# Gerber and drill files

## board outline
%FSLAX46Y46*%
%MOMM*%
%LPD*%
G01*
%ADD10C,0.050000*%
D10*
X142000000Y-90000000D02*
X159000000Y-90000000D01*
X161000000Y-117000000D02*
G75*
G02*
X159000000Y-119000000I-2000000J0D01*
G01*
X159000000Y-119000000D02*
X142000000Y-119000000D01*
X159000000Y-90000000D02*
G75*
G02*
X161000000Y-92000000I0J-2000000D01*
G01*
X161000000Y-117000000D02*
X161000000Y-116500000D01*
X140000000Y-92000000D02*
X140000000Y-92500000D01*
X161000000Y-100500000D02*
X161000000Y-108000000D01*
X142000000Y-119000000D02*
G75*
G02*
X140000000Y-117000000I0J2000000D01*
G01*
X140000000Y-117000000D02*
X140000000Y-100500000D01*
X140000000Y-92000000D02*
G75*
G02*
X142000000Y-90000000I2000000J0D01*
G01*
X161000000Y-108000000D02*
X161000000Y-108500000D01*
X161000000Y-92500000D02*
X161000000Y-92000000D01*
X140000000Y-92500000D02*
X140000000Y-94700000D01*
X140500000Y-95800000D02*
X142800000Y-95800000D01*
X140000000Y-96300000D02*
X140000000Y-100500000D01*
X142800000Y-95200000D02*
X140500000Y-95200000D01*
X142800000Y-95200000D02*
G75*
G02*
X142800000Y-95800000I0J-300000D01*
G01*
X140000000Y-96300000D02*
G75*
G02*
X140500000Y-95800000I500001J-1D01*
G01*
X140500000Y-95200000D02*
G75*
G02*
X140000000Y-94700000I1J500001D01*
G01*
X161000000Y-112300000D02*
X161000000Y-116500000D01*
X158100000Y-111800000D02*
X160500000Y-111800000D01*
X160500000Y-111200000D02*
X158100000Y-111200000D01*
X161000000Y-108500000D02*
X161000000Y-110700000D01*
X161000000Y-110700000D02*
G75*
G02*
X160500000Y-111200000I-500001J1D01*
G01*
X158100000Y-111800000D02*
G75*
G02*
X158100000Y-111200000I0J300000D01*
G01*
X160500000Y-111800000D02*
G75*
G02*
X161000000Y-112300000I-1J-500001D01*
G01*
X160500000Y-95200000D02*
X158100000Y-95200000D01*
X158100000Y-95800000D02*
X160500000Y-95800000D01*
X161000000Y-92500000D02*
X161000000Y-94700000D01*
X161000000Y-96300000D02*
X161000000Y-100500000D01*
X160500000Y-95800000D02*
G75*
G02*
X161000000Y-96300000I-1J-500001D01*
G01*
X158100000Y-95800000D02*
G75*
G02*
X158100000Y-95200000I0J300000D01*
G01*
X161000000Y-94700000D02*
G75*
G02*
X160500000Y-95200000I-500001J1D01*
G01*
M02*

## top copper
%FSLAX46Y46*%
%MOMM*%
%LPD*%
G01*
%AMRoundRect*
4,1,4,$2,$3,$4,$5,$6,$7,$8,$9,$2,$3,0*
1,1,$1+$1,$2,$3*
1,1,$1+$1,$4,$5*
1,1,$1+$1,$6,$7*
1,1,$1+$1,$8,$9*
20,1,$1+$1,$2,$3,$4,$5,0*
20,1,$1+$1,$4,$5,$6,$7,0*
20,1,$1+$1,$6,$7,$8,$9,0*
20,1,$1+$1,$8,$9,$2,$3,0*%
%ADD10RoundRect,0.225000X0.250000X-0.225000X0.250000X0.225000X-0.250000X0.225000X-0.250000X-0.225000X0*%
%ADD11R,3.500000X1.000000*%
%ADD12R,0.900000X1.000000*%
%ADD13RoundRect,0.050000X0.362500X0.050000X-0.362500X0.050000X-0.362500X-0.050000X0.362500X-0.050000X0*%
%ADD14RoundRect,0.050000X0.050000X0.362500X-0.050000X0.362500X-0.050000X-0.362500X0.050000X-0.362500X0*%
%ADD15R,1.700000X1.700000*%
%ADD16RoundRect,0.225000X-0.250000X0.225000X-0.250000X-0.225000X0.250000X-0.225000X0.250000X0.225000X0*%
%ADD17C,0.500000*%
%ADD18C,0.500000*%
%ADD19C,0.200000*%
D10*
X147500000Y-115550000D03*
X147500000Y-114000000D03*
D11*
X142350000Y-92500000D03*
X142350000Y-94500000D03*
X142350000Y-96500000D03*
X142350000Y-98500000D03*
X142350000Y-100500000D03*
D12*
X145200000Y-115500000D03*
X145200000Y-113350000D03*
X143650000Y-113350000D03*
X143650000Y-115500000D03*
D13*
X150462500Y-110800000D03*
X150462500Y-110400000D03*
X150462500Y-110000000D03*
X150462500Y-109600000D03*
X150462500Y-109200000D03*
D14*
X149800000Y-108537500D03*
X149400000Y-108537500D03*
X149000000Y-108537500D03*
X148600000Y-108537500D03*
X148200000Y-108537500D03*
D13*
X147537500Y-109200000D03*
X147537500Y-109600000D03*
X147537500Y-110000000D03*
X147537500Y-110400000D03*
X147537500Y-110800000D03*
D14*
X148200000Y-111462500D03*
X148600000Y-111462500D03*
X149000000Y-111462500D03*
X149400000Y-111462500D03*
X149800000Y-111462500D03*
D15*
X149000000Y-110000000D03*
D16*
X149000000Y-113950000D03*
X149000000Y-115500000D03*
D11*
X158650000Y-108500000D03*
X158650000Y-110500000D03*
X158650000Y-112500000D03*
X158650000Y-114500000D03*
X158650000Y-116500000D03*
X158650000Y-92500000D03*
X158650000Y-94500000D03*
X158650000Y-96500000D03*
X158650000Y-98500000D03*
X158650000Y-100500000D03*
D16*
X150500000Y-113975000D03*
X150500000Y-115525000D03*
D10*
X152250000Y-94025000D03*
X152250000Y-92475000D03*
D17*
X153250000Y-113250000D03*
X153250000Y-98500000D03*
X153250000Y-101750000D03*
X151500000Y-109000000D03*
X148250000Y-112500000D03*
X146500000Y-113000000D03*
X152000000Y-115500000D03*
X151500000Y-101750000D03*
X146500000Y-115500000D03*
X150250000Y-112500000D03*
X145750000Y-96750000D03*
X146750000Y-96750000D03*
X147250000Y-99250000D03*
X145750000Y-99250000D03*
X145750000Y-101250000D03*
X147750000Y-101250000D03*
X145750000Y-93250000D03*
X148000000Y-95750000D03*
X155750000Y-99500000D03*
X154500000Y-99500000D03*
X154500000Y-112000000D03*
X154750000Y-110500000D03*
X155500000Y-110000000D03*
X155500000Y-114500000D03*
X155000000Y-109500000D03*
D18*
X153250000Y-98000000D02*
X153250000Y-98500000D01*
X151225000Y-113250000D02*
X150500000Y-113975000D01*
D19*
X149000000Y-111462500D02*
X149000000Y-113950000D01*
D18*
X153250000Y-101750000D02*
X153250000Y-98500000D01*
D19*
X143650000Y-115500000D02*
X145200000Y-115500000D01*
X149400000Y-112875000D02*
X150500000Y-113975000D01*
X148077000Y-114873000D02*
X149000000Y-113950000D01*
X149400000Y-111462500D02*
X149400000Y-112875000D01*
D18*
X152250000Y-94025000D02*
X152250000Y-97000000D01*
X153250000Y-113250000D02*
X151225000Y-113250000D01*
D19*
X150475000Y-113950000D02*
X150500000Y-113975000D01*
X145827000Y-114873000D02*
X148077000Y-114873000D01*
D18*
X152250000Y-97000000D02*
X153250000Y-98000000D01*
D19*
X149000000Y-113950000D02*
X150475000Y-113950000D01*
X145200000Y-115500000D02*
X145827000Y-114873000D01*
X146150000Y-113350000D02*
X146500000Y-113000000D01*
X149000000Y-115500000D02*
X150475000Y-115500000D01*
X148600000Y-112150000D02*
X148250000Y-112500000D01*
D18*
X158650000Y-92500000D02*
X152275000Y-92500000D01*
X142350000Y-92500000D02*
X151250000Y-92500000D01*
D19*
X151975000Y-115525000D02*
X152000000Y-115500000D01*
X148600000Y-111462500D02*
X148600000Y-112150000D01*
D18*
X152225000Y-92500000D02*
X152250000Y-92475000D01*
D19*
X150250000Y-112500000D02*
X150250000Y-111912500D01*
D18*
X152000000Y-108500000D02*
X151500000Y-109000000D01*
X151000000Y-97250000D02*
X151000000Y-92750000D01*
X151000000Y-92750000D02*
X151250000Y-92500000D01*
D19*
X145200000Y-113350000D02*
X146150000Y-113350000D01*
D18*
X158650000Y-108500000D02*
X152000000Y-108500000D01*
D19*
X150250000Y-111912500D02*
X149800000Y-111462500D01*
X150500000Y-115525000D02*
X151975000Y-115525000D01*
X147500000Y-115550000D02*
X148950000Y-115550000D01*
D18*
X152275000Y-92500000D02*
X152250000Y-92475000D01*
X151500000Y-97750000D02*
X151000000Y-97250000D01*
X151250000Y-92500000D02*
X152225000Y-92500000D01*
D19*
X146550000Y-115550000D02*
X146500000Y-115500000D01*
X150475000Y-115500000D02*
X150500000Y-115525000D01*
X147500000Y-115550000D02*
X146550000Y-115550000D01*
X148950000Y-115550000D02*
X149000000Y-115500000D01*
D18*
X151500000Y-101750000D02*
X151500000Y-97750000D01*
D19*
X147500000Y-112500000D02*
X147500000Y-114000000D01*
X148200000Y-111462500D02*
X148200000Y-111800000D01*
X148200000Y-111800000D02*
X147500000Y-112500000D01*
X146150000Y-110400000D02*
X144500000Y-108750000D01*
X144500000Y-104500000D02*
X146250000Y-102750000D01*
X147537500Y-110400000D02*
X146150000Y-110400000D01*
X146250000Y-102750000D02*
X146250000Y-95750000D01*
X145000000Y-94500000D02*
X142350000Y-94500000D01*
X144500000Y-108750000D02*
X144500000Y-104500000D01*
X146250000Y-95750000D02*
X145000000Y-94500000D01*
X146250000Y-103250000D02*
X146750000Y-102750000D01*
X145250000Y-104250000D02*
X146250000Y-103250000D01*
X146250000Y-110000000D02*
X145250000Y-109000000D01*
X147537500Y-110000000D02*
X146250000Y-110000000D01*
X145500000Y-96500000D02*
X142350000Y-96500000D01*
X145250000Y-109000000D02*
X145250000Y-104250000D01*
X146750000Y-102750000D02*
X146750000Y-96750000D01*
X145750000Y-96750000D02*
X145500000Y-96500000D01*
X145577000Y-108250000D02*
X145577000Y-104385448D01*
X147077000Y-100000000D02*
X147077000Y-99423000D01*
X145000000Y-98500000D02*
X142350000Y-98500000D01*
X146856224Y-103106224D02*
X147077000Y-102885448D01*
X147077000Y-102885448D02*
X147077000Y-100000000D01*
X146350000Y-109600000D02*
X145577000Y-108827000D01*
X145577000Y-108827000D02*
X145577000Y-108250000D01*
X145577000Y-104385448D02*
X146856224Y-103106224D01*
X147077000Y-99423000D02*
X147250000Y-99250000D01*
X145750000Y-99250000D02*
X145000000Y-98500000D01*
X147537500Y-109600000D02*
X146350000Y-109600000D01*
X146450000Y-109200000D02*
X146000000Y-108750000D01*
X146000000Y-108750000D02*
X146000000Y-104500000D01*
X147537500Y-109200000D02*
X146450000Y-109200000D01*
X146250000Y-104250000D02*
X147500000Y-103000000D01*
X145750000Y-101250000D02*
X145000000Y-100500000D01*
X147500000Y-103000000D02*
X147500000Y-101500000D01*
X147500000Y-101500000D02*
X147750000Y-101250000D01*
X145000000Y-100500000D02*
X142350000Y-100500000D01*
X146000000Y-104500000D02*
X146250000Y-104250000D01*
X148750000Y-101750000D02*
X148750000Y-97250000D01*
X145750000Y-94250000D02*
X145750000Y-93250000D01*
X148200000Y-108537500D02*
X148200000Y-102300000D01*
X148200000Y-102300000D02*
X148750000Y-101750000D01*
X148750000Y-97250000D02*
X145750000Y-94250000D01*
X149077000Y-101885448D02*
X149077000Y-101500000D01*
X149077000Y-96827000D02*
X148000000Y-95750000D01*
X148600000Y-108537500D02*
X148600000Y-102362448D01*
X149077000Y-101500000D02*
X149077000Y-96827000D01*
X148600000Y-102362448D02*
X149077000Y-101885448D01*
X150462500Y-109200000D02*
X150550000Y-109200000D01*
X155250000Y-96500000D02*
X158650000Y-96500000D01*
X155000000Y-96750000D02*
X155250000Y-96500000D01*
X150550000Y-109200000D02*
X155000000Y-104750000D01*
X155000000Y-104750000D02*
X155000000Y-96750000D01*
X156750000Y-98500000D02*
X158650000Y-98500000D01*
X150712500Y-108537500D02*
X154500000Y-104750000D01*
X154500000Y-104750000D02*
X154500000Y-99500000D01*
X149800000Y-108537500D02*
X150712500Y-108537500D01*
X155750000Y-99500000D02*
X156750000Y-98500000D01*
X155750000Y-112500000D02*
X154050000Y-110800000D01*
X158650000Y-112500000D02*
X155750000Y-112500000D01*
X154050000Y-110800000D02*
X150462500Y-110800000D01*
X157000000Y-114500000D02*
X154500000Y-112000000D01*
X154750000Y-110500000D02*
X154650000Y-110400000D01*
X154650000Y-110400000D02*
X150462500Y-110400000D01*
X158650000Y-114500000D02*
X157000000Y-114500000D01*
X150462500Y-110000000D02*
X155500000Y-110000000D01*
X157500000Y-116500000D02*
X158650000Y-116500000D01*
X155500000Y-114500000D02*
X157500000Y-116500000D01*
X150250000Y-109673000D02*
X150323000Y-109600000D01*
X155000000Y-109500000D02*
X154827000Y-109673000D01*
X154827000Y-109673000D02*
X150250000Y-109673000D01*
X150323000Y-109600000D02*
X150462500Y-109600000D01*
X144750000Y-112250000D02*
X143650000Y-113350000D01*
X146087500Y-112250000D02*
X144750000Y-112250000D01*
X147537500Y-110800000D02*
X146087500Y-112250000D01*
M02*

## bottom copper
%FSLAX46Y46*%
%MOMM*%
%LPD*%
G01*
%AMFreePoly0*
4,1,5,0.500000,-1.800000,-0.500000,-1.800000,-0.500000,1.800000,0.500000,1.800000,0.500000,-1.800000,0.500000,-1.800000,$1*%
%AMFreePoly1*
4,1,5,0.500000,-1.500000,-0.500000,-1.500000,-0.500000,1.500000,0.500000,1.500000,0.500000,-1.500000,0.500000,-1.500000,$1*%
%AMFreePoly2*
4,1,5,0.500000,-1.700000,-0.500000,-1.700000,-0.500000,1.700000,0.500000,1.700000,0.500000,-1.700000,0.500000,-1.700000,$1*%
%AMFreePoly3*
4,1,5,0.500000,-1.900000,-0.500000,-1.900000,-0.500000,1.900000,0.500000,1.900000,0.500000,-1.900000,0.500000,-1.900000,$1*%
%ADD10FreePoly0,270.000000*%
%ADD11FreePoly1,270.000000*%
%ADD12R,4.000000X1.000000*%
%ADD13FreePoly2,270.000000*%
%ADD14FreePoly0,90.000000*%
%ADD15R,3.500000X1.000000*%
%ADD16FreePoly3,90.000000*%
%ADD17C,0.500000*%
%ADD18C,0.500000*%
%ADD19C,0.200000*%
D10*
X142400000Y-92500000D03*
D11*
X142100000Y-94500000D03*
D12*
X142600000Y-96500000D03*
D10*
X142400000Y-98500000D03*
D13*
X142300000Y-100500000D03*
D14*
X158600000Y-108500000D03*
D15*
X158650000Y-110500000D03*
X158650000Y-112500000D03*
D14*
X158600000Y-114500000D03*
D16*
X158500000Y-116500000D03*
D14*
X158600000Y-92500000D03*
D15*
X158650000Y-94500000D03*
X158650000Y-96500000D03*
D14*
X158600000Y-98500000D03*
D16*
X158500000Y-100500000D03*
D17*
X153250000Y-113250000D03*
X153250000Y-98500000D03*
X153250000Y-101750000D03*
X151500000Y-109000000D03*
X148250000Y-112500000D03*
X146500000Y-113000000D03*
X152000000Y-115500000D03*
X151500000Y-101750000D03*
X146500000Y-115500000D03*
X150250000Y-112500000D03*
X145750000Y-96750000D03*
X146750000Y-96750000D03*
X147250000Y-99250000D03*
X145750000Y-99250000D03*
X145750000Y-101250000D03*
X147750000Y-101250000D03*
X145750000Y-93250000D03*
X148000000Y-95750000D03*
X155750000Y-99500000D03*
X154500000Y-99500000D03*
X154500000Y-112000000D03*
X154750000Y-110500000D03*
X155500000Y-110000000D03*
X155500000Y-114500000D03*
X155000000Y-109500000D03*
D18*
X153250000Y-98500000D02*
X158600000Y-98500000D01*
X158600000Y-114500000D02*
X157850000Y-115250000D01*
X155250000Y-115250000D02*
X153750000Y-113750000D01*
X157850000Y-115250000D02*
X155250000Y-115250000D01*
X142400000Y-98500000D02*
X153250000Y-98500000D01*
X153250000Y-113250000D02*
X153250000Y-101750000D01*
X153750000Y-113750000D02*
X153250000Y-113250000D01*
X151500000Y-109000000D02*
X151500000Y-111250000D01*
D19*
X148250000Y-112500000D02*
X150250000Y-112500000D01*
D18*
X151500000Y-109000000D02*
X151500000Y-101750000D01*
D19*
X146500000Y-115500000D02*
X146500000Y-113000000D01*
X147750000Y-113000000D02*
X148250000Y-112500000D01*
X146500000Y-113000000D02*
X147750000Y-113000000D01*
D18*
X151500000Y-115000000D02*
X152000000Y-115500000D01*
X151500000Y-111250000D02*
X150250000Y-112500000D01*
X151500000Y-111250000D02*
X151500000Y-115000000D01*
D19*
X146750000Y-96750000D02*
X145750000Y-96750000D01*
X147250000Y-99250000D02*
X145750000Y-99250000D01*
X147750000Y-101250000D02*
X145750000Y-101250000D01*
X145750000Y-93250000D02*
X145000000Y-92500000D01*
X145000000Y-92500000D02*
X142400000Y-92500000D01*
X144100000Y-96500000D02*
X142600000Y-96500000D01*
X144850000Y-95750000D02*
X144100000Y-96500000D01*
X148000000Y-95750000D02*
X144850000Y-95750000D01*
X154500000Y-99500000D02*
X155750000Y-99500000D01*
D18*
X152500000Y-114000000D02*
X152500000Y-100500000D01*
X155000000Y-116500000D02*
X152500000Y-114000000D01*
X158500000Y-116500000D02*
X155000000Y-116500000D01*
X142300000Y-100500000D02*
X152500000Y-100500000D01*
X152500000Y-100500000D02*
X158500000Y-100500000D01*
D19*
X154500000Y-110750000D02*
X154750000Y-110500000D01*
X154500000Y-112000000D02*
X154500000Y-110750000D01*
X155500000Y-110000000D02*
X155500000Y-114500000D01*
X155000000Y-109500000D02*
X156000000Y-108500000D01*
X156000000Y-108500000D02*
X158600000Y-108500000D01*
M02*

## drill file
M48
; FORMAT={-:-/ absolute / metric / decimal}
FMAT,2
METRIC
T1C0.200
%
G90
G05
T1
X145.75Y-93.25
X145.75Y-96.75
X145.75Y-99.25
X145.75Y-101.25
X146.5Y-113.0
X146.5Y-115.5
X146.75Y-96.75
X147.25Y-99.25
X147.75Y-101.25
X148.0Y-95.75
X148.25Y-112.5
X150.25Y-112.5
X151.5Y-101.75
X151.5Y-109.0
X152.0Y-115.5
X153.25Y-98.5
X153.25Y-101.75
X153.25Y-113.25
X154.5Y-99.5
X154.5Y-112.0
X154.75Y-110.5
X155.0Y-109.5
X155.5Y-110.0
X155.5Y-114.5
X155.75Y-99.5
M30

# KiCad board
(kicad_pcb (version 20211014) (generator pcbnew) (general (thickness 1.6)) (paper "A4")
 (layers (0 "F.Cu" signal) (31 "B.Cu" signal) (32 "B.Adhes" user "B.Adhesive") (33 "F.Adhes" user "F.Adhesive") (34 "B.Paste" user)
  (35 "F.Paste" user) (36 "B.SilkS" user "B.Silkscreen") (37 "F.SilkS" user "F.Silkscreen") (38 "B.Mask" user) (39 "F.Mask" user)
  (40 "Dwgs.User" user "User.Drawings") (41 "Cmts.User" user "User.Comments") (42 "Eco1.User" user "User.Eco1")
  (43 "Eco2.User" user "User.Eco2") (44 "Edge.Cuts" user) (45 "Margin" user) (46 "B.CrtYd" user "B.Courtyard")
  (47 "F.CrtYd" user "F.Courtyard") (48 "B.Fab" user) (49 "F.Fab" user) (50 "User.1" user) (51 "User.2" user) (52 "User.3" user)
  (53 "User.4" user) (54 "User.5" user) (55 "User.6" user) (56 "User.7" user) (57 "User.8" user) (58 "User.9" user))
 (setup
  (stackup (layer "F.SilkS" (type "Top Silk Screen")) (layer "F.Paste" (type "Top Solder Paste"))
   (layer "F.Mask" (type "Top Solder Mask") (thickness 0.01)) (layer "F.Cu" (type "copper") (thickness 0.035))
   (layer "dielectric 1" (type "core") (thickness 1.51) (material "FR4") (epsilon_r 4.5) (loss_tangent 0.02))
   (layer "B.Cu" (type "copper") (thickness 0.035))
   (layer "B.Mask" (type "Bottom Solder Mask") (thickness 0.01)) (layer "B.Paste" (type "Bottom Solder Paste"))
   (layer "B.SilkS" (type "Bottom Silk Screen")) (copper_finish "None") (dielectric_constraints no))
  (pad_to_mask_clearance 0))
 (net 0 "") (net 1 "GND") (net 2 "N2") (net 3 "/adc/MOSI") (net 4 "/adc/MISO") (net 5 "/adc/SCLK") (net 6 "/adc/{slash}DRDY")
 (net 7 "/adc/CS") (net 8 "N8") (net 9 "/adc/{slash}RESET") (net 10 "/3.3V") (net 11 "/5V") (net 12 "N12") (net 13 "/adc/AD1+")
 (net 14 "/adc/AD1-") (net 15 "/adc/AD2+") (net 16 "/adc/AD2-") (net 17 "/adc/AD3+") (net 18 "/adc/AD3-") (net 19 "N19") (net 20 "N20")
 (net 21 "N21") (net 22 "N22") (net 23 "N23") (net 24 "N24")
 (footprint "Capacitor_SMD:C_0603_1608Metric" (layer "F.Cu") (at 147.5 114.775 90)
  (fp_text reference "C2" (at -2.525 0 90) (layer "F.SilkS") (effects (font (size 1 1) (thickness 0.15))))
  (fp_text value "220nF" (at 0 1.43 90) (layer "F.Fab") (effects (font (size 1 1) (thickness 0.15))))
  (pad "1" smd roundrect (at -0.775 0 90) (size 0.9 0.95) (layers "F.Cu" "F.Paste" "F.Mask") (roundrect_rratio 0.25) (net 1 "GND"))
  (pad "2" smd roundrect (at 0.775 0 90) (size 0.9 0.95) (layers "F.Cu" "F.Paste" "F.Mask") (roundrect_rratio 0.25) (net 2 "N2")))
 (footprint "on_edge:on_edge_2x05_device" (layer "F.Cu") (at 140 96.5 -90)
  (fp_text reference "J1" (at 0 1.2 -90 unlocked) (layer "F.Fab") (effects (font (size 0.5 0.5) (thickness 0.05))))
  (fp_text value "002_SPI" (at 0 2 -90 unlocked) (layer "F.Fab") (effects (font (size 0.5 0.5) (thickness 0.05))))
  (fp_line (start -4 0) (end -1.8 0) (layer "Edge.Cuts") (width 0.05))
  (fp_line (start -0.7 -0.5) (end -0.7 -2.8) (layer "Edge.Cuts") (width 0.05))
  (fp_line (start -0.2 0) (end 4 0) (layer "Edge.Cuts") (width 0.05))
  (fp_line (start -1.3 -2.8) (end -1.3 -0.5) (layer "Edge.Cuts") (width 0.05))
  (fp_arc (start -1.3 -2.8) (mid -1 -3.1) (end -0.7 -2.8) (layer "Edge.Cuts") (width 0.05))
  (fp_arc (start -0.2 0) (mid -0.553553 -0.146447) (end -0.7 -0.5) (layer "Edge.Cuts") (width 0.05))
  (fp_arc (start -1.3 -0.5) (mid -1.446447 -0.146447) (end -1.8 0) (layer "Edge.Cuts") (width 0.05))
  (pad "1" smd rect (at -4 -2.35 90) (size 1 3.5) (layers "F.Cu" "F.Mask") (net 1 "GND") (zone_connect 0))
  (pad "2" smd rect (at -2 -2.35 270) (size 1 3.5) (layers "F.Cu" "F.Mask") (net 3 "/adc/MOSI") (zone_connect 0))
  (pad "3" smd rect (at 0 -2.35 270) (size 1 3.5) (layers "F.Cu" "F.Mask") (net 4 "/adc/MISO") (zone_connect 0))
  (pad "4" smd rect (at 2 -2.35 90) (size 1 3.5) (layers "F.Cu" "F.Mask") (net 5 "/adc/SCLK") (zone_connect 0))
  (pad "5" smd rect (at 4 -2.35 90) (size 1 3.5) (layers "F.Cu" "F.Mask") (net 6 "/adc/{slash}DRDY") (zone_connect 0))
  (pad "6" smd custom (at -4 -2.4 270) (size 1 3.6) (layers "B.Cu" "B.Mask") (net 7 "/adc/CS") (zone_connect 0)
   (options (clearance outline) (anchor rect)) (primitives))
  (pad "7" smd custom (at -2 -2.1 270) (size 1 3) (layers "B.Cu" "B.Mask") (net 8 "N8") (zone_connect 0)
   (options (clearance outline) (anchor rect)) (primitives))
  (pad "8" smd rect (at 0 -2.6 270) (size 1 4) (layers "B.Cu" "B.Mask") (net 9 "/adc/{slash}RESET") (zone_connect 0))
  (pad "9" smd custom (at 2 -2.4 270) (size 1 3.6) (layers "B.Cu" "B.Mask") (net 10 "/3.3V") (zone_connect 0)
   (options (clearance outline) (anchor rect)) (primitives))
  (pad "10" smd custom (at 4 -2.3 270) (size 1 3.4) (layers "B.Cu" "B.Mask") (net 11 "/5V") (zone_connect 0)
   (options (clearance outline) (anchor rect)) (primitives)))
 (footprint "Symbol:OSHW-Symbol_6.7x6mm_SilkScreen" (layer "F.Cu") (at 143.4 108.6)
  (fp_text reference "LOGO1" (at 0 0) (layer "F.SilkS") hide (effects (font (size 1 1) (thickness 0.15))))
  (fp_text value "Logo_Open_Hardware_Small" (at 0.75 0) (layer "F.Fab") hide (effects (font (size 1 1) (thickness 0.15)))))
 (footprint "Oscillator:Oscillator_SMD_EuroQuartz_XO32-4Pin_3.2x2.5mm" (layer "F.Cu") (at 144.425 114.425 180)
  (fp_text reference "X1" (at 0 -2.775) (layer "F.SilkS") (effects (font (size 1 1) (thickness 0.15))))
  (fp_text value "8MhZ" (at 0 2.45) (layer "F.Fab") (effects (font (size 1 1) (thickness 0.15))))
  (pad "1" smd rect (at -0.775 -1.075 90) (size 1 0.9) (layers "F.Cu" "F.Paste" "F.Mask") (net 10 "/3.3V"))
  (pad "2" smd rect (at -0.775 1.075 90) (size 1 0.9) (layers "F.Cu" "F.Paste" "F.Mask") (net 1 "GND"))
  (pad "3" smd rect (at 0.775 1.075 90) (size 1 0.9) (layers "F.Cu" "F.Paste" "F.Mask") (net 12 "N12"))
  (pad "4" smd rect (at 0.775 -1.075 90) (size 1 0.9) (layers "F.Cu" "F.Paste" "F.Mask") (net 10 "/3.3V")))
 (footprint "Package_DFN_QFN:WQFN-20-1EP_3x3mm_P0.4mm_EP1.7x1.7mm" (layer "F.Cu") (at 149 110 180)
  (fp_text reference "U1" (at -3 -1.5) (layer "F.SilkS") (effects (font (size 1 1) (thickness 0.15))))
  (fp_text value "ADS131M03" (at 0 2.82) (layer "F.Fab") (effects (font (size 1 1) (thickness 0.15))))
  (pad "" smd roundrect (at -0.425 0.425 180) (size 0.69 0.69) (layers "F.Paste") (roundrect_rratio 0.25))
  (pad "" smd roundrect (at 0.425 0.425 180) (size 0.69 0.69) (layers "F.Paste") (roundrect_rratio 0.25))
  (pad "" smd roundrect (at -0.425 -0.425 180) (size 0.69 0.69) (layers "F.Paste") (roundrect_rratio 0.25))
  (pad "" smd roundrect (at 0.425 -0.425 180) (size 0.69 0.69) (layers "F.Paste") (roundrect_rratio 0.25))
  (pad "1" smd roundrect (at -1.4625 -0.8 180) (size 0.825 0.2) (layers "F.Cu" "F.Paste" "F.Mask") (roundrect_rratio 0.25)
   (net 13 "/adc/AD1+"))
  (pad "2" smd roundrect (at -1.4625 -0.4 180) (size 0.825 0.2) (layers "F.Cu" "F.Paste" "F.Mask") (roundrect_rratio 0.25)
   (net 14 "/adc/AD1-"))
  (pad "3" smd roundrect (at -1.4625 0 180) (size 0.825 0.2) (layers "F.Cu" "F.Paste" "F.Mask") (roundrect_rratio 0.25) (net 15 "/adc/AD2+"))
  (pad "4" smd roundrect (at -1.4625 0.4 180) (size 0.825 0.2) (layers "F.Cu" "F.Paste" "F.Mask") (roundrect_rratio 0.25)
   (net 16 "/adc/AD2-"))
  (pad "5" smd roundrect (at -1.4625 0.8 180) (size 0.825 0.2) (layers "F.Cu" "F.Paste" "F.Mask") (roundrect_rratio 0.25)
   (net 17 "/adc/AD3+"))
  (pad "6" smd roundrect (at -0.8 1.4625 180) (size 0.2 0.825) (layers "F.Cu" "F.Paste" "F.Mask") (roundrect_rratio 0.25)
   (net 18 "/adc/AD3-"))
  (pad "7" smd roundrect (at -0.4 1.4625 180) (size 0.2 0.825) (layers "F.Cu" "F.Paste" "F.Mask") (roundrect_rratio 0.25) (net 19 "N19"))
  (pad "8" smd roundrect (at 0 1.4625 180) (size 0.2 0.825) (layers "F.Cu" "F.Paste" "F.Mask") (roundrect_rratio 0.25) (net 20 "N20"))
  (pad "9" smd roundrect (at 0.4 1.4625 180) (size 0.2 0.825) (layers "F.Cu" "F.Paste" "F.Mask") (roundrect_rratio 0.25)
   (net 9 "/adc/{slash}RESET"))
  (pad "10" smd roundrect (at 0.8 1.4625 180) (size 0.2 0.825) (layers "F.Cu" "F.Paste" "F.Mask") (roundrect_rratio 0.25) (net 7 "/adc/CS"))
  (pad "11" smd roundrect (at 1.4625 0.8 180) (size 0.825 0.2) (layers "F.Cu" "F.Paste" "F.Mask") (roundrect_rratio 0.25)
   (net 6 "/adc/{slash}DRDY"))
  (pad "12" smd roundrect (at 1.4625 0.4 180) (size 0.825 0.2) (layers "F.Cu" "F.Paste" "F.Mask") (roundrect_rratio 0.25)
   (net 5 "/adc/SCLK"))
  (pad "13" smd roundrect (at 1.4625 0 180) (size 0.825 0.2) (layers "F.Cu" "F.Paste" "F.Mask") (roundrect_rratio 0.25) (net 4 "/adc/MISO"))
  (pad "14" smd roundrect (at 1.4625 -0.4 180) (size 0.825 0.2) (layers "F.Cu" "F.Paste" "F.Mask") (roundrect_rratio 0.25)
   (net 3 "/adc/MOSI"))
  (pad "15" smd roundrect (at 1.4625 -0.8 180) (size 0.825 0.2) (layers "F.Cu" "F.Paste" "F.Mask") (roundrect_rratio 0.25) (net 12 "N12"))
  (pad "16" smd roundrect (at 0.8 -1.4625 180) (size 0.2 0.825) (layers "F.Cu" "F.Paste" "F.Mask") (roundrect_rratio 0.25) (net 2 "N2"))
  (pad "17" smd roundrect (at 0.4 -1.4625 180) (size 0.2 0.825) (layers "F.Cu" "F.Paste" "F.Mask") (roundrect_rratio 0.25) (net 1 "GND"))
  (pad "18" smd roundrect (at 0 -1.4625 180) (size 0.2 0.825) (layers "F.Cu" "F.Paste" "F.Mask") (roundrect_rratio 0.25) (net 10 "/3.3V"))
  (pad "19" smd roundrect (at -0.4 -1.4625 180) (size 0.2 0.825) (layers "F.Cu" "F.Paste" "F.Mask") (roundrect_rratio 0.25) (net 10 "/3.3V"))
  (pad "20" smd roundrect (at -0.8 -1.4625 180) (size 0.2 0.825) (layers "F.Cu" "F.Paste" "F.Mask") (roundrect_rratio 0.25) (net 1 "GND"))
  (pad "21" smd rect (at 0 0 180) (size 1.7 1.7) (layers "F.Cu" "F.Mask")))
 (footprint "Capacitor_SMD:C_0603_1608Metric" (layer "F.Cu") (at 149 114.725 -90)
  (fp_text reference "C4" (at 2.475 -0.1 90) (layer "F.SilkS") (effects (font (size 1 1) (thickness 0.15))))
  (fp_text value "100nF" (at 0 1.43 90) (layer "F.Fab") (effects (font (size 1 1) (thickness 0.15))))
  (pad "1" smd roundrect (at -0.775 0 270) (size 0.9 0.95) (layers "F.Cu" "F.Paste" "F.Mask") (roundrect_rratio 0.25) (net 10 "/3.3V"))
  (pad "2" smd roundrect (at 0.775 0 270) (size 0.9 0.95) (layers "F.Cu" "F.Paste" "F.Mask") (roundrect_rratio 0.25) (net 1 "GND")))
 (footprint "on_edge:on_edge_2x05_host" (layer "F.Cu") (at 161 112.5 -90)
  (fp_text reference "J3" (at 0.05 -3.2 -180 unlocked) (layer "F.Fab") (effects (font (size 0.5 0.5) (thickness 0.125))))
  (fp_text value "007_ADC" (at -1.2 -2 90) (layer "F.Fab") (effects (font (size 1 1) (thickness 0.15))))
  (fp_line (start -0.2 0) (end 4 0) (layer "Edge.Cuts") (width 0.05))
  (fp_line (start -0.7 2.9) (end -0.7 0.5) (layer "Edge.Cuts") (width 0.05))
  (fp_line (start -1.3 0.5) (end -1.3 2.9) (layer "Edge.Cuts") (width 0.05))
  (fp_line (start -4 0) (end -1.8 0) (layer "Edge.Cuts") (width 0.05))
  (fp_arc (start -1.8 0) (mid -1.446447 0.146447) (end -1.3 0.5) (layer "Edge.Cuts") (width 0.05))
  (fp_arc (start -0.7 2.9) (mid -1 3.2) (end -1.3 2.9) (layer "Edge.Cuts") (width 0.05))
  (fp_arc (start -0.7 0.5) (mid -0.553553 0.146447) (end -0.2 0) (layer "Edge.Cuts") (width 0.05))
  (pad "1" smd rect (at -4 2.35 270) (size 1 3.5) (layers "F.Cu" "F.Mask") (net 1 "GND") (zone_connect 0))
  (pad "2" smd rect (at -2 2.35 270) (size 1 3.5) (layers "F.Cu" "F.Mask") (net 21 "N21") (zone_connect 0))
  (pad "3" smd rect (at 0 2.35 270) (size 1 3.5) (layers "F.Cu" "F.Mask") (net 13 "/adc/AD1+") (zone_connect 0))
  (pad "4" smd rect (at 2 2.35 270) (size 1 3.5) (layers "F.Cu" "F.Mask") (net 14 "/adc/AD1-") (zone_connect 0))
  (pad "5" smd rect (at 4 2.35 270) (size 1 3.5) (layers "F.Cu" "F.Mask") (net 15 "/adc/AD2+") (zone_connect 0))
  (pad "6" smd custom (at -4 2.4 90) (size 1 3.6) (layers "B.Cu" "B.Mask") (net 16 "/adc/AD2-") (zone_connect 0)
   (options (clearance outline) (anchor rect)) (primitives))
  (pad "7" smd rect (at -2 2.35 90) (size 1 3.5) (layers "B.Cu" "B.Mask") (zone_connect 0))
  (pad "8" smd rect (at 0 2.35 90) (size 1 3.5) (layers "B.Cu" "B.Mask") (zone_connect 0))
  (pad "9" smd custom (at 2 2.4 90) (size 1 3.6) (layers "B.Cu" "B.Mask") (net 10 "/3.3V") (zone_connect 0)
   (options (clearance outline) (anchor rect)) (primitives))
  (pad "10" smd custom (at 4 2.5 90) (size 1 3.8) (layers "B.Cu" "B.Mask") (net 11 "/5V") (zone_connect 0)
   (options (clearance outline) (anchor rect)) (primitives)))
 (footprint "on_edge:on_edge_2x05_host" (layer "F.Cu") (at 161 96.5 -90)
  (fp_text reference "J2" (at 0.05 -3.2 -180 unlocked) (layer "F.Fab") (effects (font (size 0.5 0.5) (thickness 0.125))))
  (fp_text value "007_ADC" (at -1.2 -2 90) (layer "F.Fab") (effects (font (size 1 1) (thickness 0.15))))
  (fp_line (start -1.3 0.5) (end -1.3 2.9) (layer "Edge.Cuts") (width 0.05))
  (fp_line (start -0.7 2.9) (end -0.7 0.5) (layer "Edge.Cuts") (width 0.05))
  (fp_line (start -4 0) (end -1.8 0) (layer "Edge.Cuts") (width 0.05))
  (fp_line (start -0.2 0) (end 4 0) (layer "Edge.Cuts") (width 0.05))
  (fp_arc (start -0.7 0.5) (mid -0.553553 0.146447) (end -0.2 0) (layer "Edge.Cuts") (width 0.05))
  (fp_arc (start -0.7 2.9) (mid -1 3.2) (end -1.3 2.9) (layer "Edge.Cuts") (width 0.05))
  (fp_arc (start -1.8 0) (mid -1.446447 0.146447) (end -1.3 0.5) (layer "Edge.Cuts") (width 0.05))
  (pad "1" smd rect (at -4 2.35 270) (size 1 3.5) (layers "F.Cu" "F.Mask") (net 1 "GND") (zone_connect 0))
  (pad "2" smd rect (at -2 2.35 270) (size 1 3.5) (layers "F.Cu" "F.Mask") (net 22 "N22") (zone_connect 0))
  (pad "3" smd rect (at 0 2.35 270) (size 1 3.5) (layers "F.Cu" "F.Mask") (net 17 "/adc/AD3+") (zone_connect 0))
  (pad "4" smd rect (at 2 2.35 270) (size 1 3.5) (layers "F.Cu" "F.Mask") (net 18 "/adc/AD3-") (zone_connect 0))
  (pad "5" smd rect (at 4 2.35 270) (size 1 3.5) (layers "F.Cu" "F.Mask") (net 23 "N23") (zone_connect 0))
  (pad "6" smd custom (at -4 2.4 90) (size 1 3.6) (layers "B.Cu" "B.Mask") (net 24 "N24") (zone_connect 0)
   (options (clearance outline) (anchor rect)) (primitives))
  (pad "7" smd rect (at -2 2.35 90) (size 1 3.5) (layers "B.Cu" "B.Mask") (zone_connect 0))
  (pad "8" smd rect (at 0 2.35 90) (size 1 3.5) (layers "B.Cu" "B.Mask") (zone_connect 0))
  (pad "9" smd custom (at 2 2.4 90) (size 1 3.6) (layers "B.Cu" "B.Mask") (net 10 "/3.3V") (zone_connect 0)
   (options (clearance outline) (anchor rect)) (primitives))
  (pad "10" smd custom (at 4 2.5 90) (size 1 3.8) (layers "B.Cu" "B.Mask") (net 11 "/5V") (zone_connect 0)
   (options (clearance outline) (anchor rect)) (primitives)))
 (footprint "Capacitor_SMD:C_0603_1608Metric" (layer "F.Cu") (at 150.5 114.75 -90)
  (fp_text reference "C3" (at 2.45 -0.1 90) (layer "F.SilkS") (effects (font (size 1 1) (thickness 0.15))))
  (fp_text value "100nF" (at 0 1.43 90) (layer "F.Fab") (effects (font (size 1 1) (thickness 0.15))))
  (pad "1" smd roundrect (at -0.775 0 270) (size 0.9 0.95) (layers "F.Cu" "F.Paste" "F.Mask") (roundrect_rratio 0.25) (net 10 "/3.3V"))
  (pad "2" smd roundrect (at 0.775 0 270) (size 0.9 0.95) (layers "F.Cu" "F.Paste" "F.Mask") (roundrect_rratio 0.25) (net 1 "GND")))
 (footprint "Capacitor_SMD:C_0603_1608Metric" (layer "F.Cu") (at 152.25 93.25 90)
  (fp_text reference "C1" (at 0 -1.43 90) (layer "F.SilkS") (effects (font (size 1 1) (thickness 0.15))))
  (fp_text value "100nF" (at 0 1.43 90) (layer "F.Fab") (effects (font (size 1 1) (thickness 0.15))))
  (pad "1" smd roundrect (at -0.775 0 90) (size 0.9 0.95) (layers "F.Cu" "F.Paste" "F.Mask") (roundrect_rratio 0.25) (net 10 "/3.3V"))
  (pad "2" smd roundrect (at 0.775 0 90) (size 0.9 0.95) (layers "F.Cu" "F.Paste" "F.Mask") (roundrect_rratio 0.25) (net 1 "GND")))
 (gr_line (start 142 90) (end 159 90) (layer "Edge.Cuts") (width 0.05))
 (gr_arc (start 161 117) (mid 160.414214 118.414214) (end 159 119) (layer "Edge.Cuts") (width 0.05))
 (gr_line (start 159 119) (end 142 119) (layer "Edge.Cuts") (width 0.05))
 (gr_arc (start 159 90) (mid 160.414214 90.585786) (end 161 92) (layer "Edge.Cuts") (width 0.05))
 (gr_line (start 161 117) (end 161 116.5) (layer "Edge.Cuts") (width 0.05))
 (gr_line (start 140 92) (end 140 92.5) (layer "Edge.Cuts") (width 0.05))
 (gr_line (start 161 100.5) (end 161 108) (layer "Edge.Cuts") (width 0.05))
 (gr_arc (start 142 119) (mid 140.585786 118.414214) (end 140 117) (layer "Edge.Cuts") (width 0.05))
 (gr_line (start 140 117) (end 140 100.5) (layer "Edge.Cuts") (width 0.05))
 (gr_arc (start 140 92) (mid 140.585786 90.585786) (end 142 90) (layer "Edge.Cuts") (width 0.05))
 (gr_line (start 161 108) (end 161 108.5) (layer "Edge.Cuts") (width 0.05))
 (gr_line (start 161 92.5) (end 161 92) (layer "Edge.Cuts") (width 0.05))
 (segment (start 153.25 98) (end 153.25 98.5) (width 0.5) (layer "F.Cu") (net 10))
 (segment (start 151.225 113.25) (end 150.5 113.975) (width 0.5) (layer "F.Cu") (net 10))
 (segment (start 149 111.4625) (end 149 113.95) (width 0.2) (layer "F.Cu") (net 10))
 (segment (start 153.25 101.75) (end 153.25 98.5) (width 0.5) (layer "F.Cu") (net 10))
 (segment (start 143.65 115.5) (end 145.2 115.5) (width 0.2) (layer "F.Cu") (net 10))
 (segment (start 149.4 112.875) (end 150.5 113.975) (width 0.2) (layer "F.Cu") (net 10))
 (segment (start 148.077 114.873) (end 149 113.95) (width 0.2) (layer "F.Cu") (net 10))
 (segment (start 149.4 111.4625) (end 149.4 112.875) (width 0.2) (layer "F.Cu") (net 10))
 (segment (start 152.25 94.025) (end 152.25 97) (width 0.5) (layer "F.Cu") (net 10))
 (segment (start 153.25 113.25) (end 151.225 113.25) (width 0.5) (layer "F.Cu") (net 10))
 (segment (start 150.475 113.95) (end 150.5 113.975) (width 0.2) (layer "F.Cu") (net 10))
 (segment (start 145.827 114.873) (end 148.077 114.873) (width 0.2) (layer "F.Cu") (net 10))
 (segment (start 152.25 97) (end 153.25 98) (width 0.5) (layer "F.Cu") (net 10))
 (segment (start 149 113.95) (end 150.475 113.95) (width 0.2) (layer "F.Cu") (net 10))
 (segment (start 145.2 115.5) (end 145.827 114.873) (width 0.2) (layer "F.Cu") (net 10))
 (via (at 153.25 113.25) (size 0.5) (drill 0.2) (layers "F.Cu" "B.Cu") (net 10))
 (via (at 153.25 98.5) (size 0.5) (drill 0.2) (layers "F.Cu" "B.Cu") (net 10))
 (via (at 153.25 101.75) (size 0.5) (drill 0.2) (layers "F.Cu" "B.Cu") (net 10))
 (segment (start 153.25 98.5) (end 158.6 98.5) (width 0.5) (layer "B.Cu") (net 10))
 (segment (start 158.6 114.5) (end 157.85 115.25) (width 0.5) (layer "B.Cu") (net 10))
 (segment (start 155.25 115.25) (end 153.75 113.75) (width 0.5) (layer "B.Cu") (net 10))
 (segment (start 157.85 115.25) (end 155.25 115.25) (width 0.5) (layer "B.Cu") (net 10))
 (segment (start 142.4 98.5) (end 153.25 98.5) (width 0.5) (layer "B.Cu") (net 10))
 (segment (start 153.25 113.25) (end 153.25 101.75) (width 0.5) (layer "B.Cu") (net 10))
 (segment (start 153.75 113.75) (end 153.25 113.25) (width 0.5) (layer "B.Cu") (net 10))
 (segment (start 146.15 113.35) (end 146.5 113) (width 0.2) (layer "F.Cu") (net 1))
 (segment (start 149 115.5) (end 150.475 115.5) (width 0.2) (layer "F.Cu") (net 1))
 (segment (start 148.6 112.15) (end 148.25 112.5) (width 0.2) (layer "F.Cu") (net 1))
 (segment (start 158.65 92.5) (end 152.275 92.5) (width 0.5) (layer "F.Cu") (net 1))
 (segment (start 142.35 92.5) (end 151.25 92.5) (width 0.5) (layer "F.Cu") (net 1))
 (segment (start 151.975 115.525) (end 152 115.5) (width 0.2) (layer "F.Cu") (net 1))
 (segment (start 148.6 111.4625) (end 148.6 112.15) (width 0.2) (layer "F.Cu") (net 1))
 (segment (start 152.225 92.5) (end 152.25 92.475) (width 0.5) (layer "F.Cu") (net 1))
 (segment (start 150.25 112.5) (end 150.25 111.9125) (width 0.2) (layer "F.Cu") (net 1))
 (segment (start 152 108.5) (end 151.5 109) (width 0.5) (layer "F.Cu") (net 1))
 (segment (start 151 97.25) (end 151 92.75) (width 0.5) (layer "F.Cu") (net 1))
 (segment (start 151 92.75) (end 151.25 92.5) (width 0.5) (layer "F.Cu") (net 1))
 (segment (start 145.2 113.35) (end 146.15 113.35) (width 0.2) (layer "F.Cu") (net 1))
 (segment (start 158.65 108.5) (end 152 108.5) (width 0.5) (layer "F.Cu") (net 1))
 (segment (start 150.25 111.9125) (end 149.8 111.4625) (width 0.2) (layer "F.Cu") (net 1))
 (segment (start 150.5 115.525) (end 151.975 115.525) (width 0.2) (layer "F.Cu") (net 1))
 (segment (start 147.5 115.55) (end 148.95 115.55) (width 0.2) (layer "F.Cu") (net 1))
 (segment (start 152.275 92.5) (end 152.25 92.475) (width 0.5) (layer "F.Cu") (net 1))
 (segment (start 151.5 97.75) (end 151 97.25) (width 0.5) (layer "F.Cu") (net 1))
 (segment (start 151.25 92.5) (end 152.225 92.5) (width 0.5) (layer "F.Cu") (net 1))
 (segment (start 146.55 115.55) (end 146.5 115.5) (width 0.2) (layer "F.Cu") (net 1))
 (segment (start 150.475 115.5) (end 150.5 115.525) (width 0.2) (layer "F.Cu") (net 1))
 (segment (start 147.5 115.55) (end 146.55 115.55) (width 0.2) (layer "F.Cu") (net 1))
 (segment (start 148.95 115.55) (end 149 115.5) (width 0.2) (layer "F.Cu") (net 1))
 (segment (start 151.5 101.75) (end 151.5 97.75) (width 0.5) (layer "F.Cu") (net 1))
 (via (at 151.5 109) (size 0.5) (drill 0.2) (layers "F.Cu" "B.Cu") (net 1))
 (via (at 148.25 112.5) (size 0.5) (drill 0.2) (layers "F.Cu" "B.Cu") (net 1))
 (via (at 146.5 113) (size 0.5) (drill 0.2) (layers "F.Cu" "B.Cu") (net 1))
 (via (at 152 115.5) (size 0.5) (drill 0.2) (layers "F.Cu" "B.Cu") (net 1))
 (via (at 151.5 101.75) (size 0.5) (drill 0.2) (layers "F.Cu" "B.Cu") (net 1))
 (via (at 146.5 115.5) (size 0.5) (drill 0.2) (layers "F.Cu" "B.Cu") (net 1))
 (via (at 150.25 112.5) (size 0.5) (drill 0.2) (layers "F.Cu" "B.Cu") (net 1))
 (segment (start 151.5 109) (end 151.5 111.25) (width 0.5) (layer "B.Cu") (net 1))
 (segment (start 148.25 112.5) (end 150.25 112.5) (width 0.2) (layer "B.Cu") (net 1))
 (segment (start 151.5 109) (end 151.5 101.75) (width 0.5) (layer "B.Cu") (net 1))
 (segment (start 146.5 115.5) (end 146.5 113) (width 0.2) (layer "B.Cu") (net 1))
 (segment (start 147.75 113) (end 148.25 112.5) (width 0.2) (layer "B.Cu") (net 1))
 (segment (start 146.5 113) (end 147.75 113) (width 0.2) (layer "B.Cu") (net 1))
 (segment (start 151.5 115) (end 152 115.5) (width 0.5) (layer "B.Cu") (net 1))
 (segment (start 151.5 111.25) (end 150.25 112.5) (width 0.5) (layer "B.Cu") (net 1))
 (segment (start 151.5 111.25) (end 151.5 115) (width 0.5) (layer "B.Cu") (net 1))
 (segment (start 147.5 112.5) (end 147.5 114) (width 0.2) (layer "F.Cu") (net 2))
 (segment (start 148.2 111.4625) (end 148.2 111.8) (width 0.2) (layer "F.Cu") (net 2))
 (segment (start 148.2 111.8) (end 147.5 112.5) (width 0.2) (layer "F.Cu") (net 2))
 (segment (start 146.15 110.4) (end 144.5 108.75) (width 0.2) (layer "F.Cu") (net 3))
 (segment (start 144.5 104.5) (end 146.25 102.75) (width 0.2) (layer "F.Cu") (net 3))
 (segment (start 147.5375 110.4) (end 146.15 110.4) (width 0.2) (layer "F.Cu") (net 3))
 (segment (start 146.25 102.75) (end 146.25 95.75) (width 0.2) (layer "F.Cu") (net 3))
 (segment (start 145 94.5) (end 142.35 94.5) (width 0.2) (layer "F.Cu") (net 3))
 (segment (start 144.5 108.75) (end 144.5 104.5) (width 0.2) (layer "F.Cu") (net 3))
 (segment (start 146.25 95.75) (end 145 94.5) (width 0.2) (layer "F.Cu") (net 3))
 (segment (start 146.25 103.25) (end 146.75 102.75) (width 0.2) (layer "F.Cu") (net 4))
 (segment (start 145.25 104.25) (end 146.25 103.25) (width 0.2) (layer "F.Cu") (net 4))
 (segment (start 146.25 110) (end 145.25 109) (width 0.2) (layer "F.Cu") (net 4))
 (segment (start 147.5375 110) (end 146.25 110) (width 0.2) (layer "F.Cu") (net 4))
 (segment (start 145.5 96.5) (end 142.35 96.5) (width 0.2) (layer "F.Cu") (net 4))
 (segment (start 145.25 109) (end 145.25 104.25) (width 0.2) (layer "F.Cu") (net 4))
 (segment (start 146.75 102.75) (end 146.75 96.75) (width 0.2) (layer "F.Cu") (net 4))
 (segment (start 145.75 96.75) (end 145.5 96.5) (width 0.2) (layer "F.Cu") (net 4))
 (via (at 145.75 96.75) (size 0.5) (drill 0.2) (layers "F.Cu" "B.Cu") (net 4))
 (via (at 146.75 96.75) (size 0.5) (drill 0.2) (layers "F.Cu" "B.Cu") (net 4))
 (segment (start 146.75 96.75) (end 145.75 96.75) (width 0.2) (layer "B.Cu") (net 4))
 (segment (start 145.577 108.25) (end 145.577 104.385448) (width 0.2) (layer "F.Cu") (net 5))
 (segment (start 147.077 100) (end 147.077 99.423) (width 0.2) (layer "F.Cu") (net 5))
 (segment (start 145 98.5) (end 142.35 98.5) (width 0.2) (layer "F.Cu") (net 5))
 (segment (start 146.856224 103.106224) (end 147.077 102.885448) (width 0.2) (layer "F.Cu") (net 5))
 (segment (start 147.077 102.885448) (end 147.077 100) (width 0.2) (layer "F.Cu") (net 5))
 (segment (start 146.35 109.6) (end 145.577 108.827) (width 0.2) (layer "F.Cu") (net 5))
 (segment (start 145.577 108.827) (end 145.577 108.25) (width 0.2) (layer "F.Cu") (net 5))
 (segment (start 145.577 104.385448) (end 146.856224 103.106224) (width 0.2) (layer "F.Cu") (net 5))
 (segment (start 147.077 99.423) (end 147.25 99.25) (width 0.2) (layer "F.Cu") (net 5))
 (segment (start 145.75 99.25) (end 145 98.5) (width 0.2) (layer "F.Cu") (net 5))
 (segment (start 147.5375 109.6) (end 146.35 109.6) (width 0.2) (layer "F.Cu") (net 5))
 (via (at 147.25 99.25) (size 0.5) (drill 0.2) (layers "F.Cu" "B.Cu") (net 5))
 (via (at 145.75 99.25) (size 0.5) (drill 0.2) (layers "F.Cu" "B.Cu") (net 5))
 (segment (start 147.25 99.25) (end 145.75 99.25) (width 0.2) (layer "B.Cu") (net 5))
 (segment (start 146.45 109.2) (end 146 108.75) (width 0.2) (layer "F.Cu") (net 6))
 (segment (start 146 108.75) (end 146 104.5) (width 0.2) (layer "F.Cu") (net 6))
 (segment (start 147.5375 109.2) (end 146.45 109.2) (width 0.2) (layer "F.Cu") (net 6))
 (segment (start 146.25 104.25) (end 147.5 103) (width 0.2) (layer "F.Cu") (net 6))
 (segment (start 145.75 101.25) (end 145 100.5) (width 0.2) (layer "F.Cu") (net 6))
 (segment (start 147.5 103) (end 147.5 101.5) (width 0.2) (layer "F.Cu") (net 6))
 (segment (start 147.5 101.5) (end 147.75 101.25) (width 0.2) (layer "F.Cu") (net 6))
 (segment (start 145 100.5) (end 142.35 100.5) (width 0.2) (layer "F.Cu") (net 6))
 (segment (start 146 104.5) (end 146.25 104.25) (width 0.2) (layer "F.Cu") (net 6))
 (via (at 145.75 101.25) (size 0.5) (drill 0.2) (layers "F.Cu" "B.Cu") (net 6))
 (via (at 147.75 101.25) (size 0.5) (drill 0.2) (layers "F.Cu" "B.Cu") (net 6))
 (segment (start 147.75 101.25) (end 145.75 101.25) (width 0.2) (layer "B.Cu") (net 6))
 (segment (start 148.75 101.75) (end 148.75 97.25) (width 0.2) (layer "F.Cu") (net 7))
 (segment (start 145.75 94.25) (end 145.75 93.25) (width 0.2) (layer "F.Cu") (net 7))
 (segment (start 148.2 108.5375) (end 148.2 102.3) (width 0.2) (layer "F.Cu") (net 7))
 (segment (start 148.2 102.3) (end 148.75 101.75) (width 0.2) (layer "F.Cu") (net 7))
 (segment (start 148.75 97.25) (end 145.75 94.25) (width 0.2) (layer "F.Cu") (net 7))
 (via (at 145.75 93.25) (size 0.5) (drill 0.2) (layers "F.Cu" "B.Cu") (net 7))
 (segment (start 145.75 93.25) (end 145 92.5) (width 0.2) (layer "B.Cu") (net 7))
 (segment (start 145 92.5) (end 142.4 92.5) (width 0.2) (layer "B.Cu") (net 7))
 (segment (start 149.077 101.885448) (end 149.077 101.5) (width 0.2) (layer "F.Cu") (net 9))
 (segment (start 149.077 96.827) (end 148 95.75) (width 0.2) (layer "F.Cu") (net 9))
 (segment (start 148.6 108.5375) (end 148.6 102.362448) (width 0.2) (layer "F.Cu") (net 9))
 (segment (start 149.077 101.5) (end 149.077 96.827) (width 0.2) (layer "F.Cu") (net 9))
 (segment (start 148.6 102.362448) (end 149.077 101.885448) (width 0.2) (layer "F.Cu") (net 9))
 (via (at 148 95.75) (size 0.5) (drill 0.2) (layers "F.Cu" "B.Cu") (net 9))
 (segment (start 144.1 96.5) (end 142.6 96.5) (width 0.2) (layer "B.Cu") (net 9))
 (segment (start 144.85 95.75) (end 144.1 96.5) (width 0.2) (layer "B.Cu") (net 9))
 (segment (start 148 95.75) (end 144.85 95.75) (width 0.2) (layer "B.Cu") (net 9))
 (segment (start 150.4625 109.2) (end 150.55 109.2) (width 0.2) (layer "F.Cu") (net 17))
 (segment (start 155.25 96.5) (end 158.65 96.5) (width 0.2) (layer "F.Cu") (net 17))
 (segment (start 155 96.75) (end 155.25 96.5) (width 0.2) (layer "F.Cu") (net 17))
 (segment (start 150.55 109.2) (end 155 104.75) (width 0.2) (layer "F.Cu") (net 17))
 (segment (start 155 104.75) (end 155 96.75) (width 0.2) (layer "F.Cu") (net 17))
 (segment (start 156.75 98.5) (end 158.65 98.5) (width 0.2) (layer "F.Cu") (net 18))
 (segment (start 150.7125 108.5375) (end 154.5 104.75) (width 0.2) (layer "F.Cu") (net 18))
 (segment (start 154.5 104.75) (end 154.5 99.5) (width 0.2) (layer "F.Cu") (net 18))
 (segment (start 149.8 108.5375) (end 150.7125 108.5375) (width 0.2) (layer "F.Cu") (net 18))
 (segment (start 155.75 99.5) (end 156.75 98.5) (width 0.2) (layer "F.Cu") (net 18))
 (via (at 155.75 99.5) (size 0.5) (drill 0.2) (layers "F.Cu" "B.Cu") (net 18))
 (via (at 154.5 99.5) (size 0.5) (drill 0.2) (layers "F.Cu" "B.Cu") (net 18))
 (segment (start 154.5 99.5) (end 155.75 99.5) (width 0.2) (layer "B.Cu") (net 18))
 (segment (start 152.5 114) (end 152.5 100.5) (width 0.5) (layer "B.Cu") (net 11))
 (segment (start 155 116.5) (end 152.5 114) (width 0.5) (layer "B.Cu") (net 11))
 (segment (start 158.5 116.5) (end 155 116.5) (width 0.5) (layer "B.Cu") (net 11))
 (segment (start 142.3 100.5) (end 152.5 100.5) (width 0.5) (layer "B.Cu") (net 11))
 (segment (start 152.5 100.5) (end 158.5 100.5) (width 0.5) (layer "B.Cu") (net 11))
 (segment (start 155.75 112.5) (end 154.05 110.8) (width 0.2) (layer "F.Cu") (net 13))
 (segment (start 158.65 112.5) (end 155.75 112.5) (width 0.2) (layer "F.Cu") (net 13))
 (segment (start 154.05 110.8) (end 150.4625 110.8) (width 0.2) (layer "F.Cu") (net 13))
 (segment (start 157 114.5) (end 154.5 112) (width 0.2) (layer "F.Cu") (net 14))
 (segment (start 154.75 110.5) (end 154.65 110.4) (width 0.2) (layer "F.Cu") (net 14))
 (segment (start 154.65 110.4) (end 150.4625 110.4) (width 0.2) (layer "F.Cu") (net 14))
 (segment (start 158.65 114.5) (end 157 114.5) (width 0.2) (layer "F.Cu") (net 14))
 (via (at 154.5 112) (size 0.5) (drill 0.2) (layers "F.Cu" "B.Cu") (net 14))
 (via (at 154.75 110.5) (size 0.5) (drill 0.2) (layers "F.Cu" "B.Cu") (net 14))
 (segment (start 154.5 110.75) (end 154.75 110.5) (width 0.2) (layer "B.Cu") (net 14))
 (segment (start 154.5 112) (end 154.5 110.75) (width 0.2) (layer "B.Cu") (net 14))
 (segment (start 150.4625 110) (end 155.5 110) (width 0.2) (layer "F.Cu") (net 15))
 (segment (start 157.5 116.5) (end 158.65 116.5) (width 0.2) (layer "F.Cu") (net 15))
 (segment (start 155.5 114.5) (end 157.5 116.5) (width 0.2) (layer "F.Cu") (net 15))
 (via (at 155.5 110) (size 0.5) (drill 0.2) (layers "F.Cu" "B.Cu") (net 15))
 (via (at 155.5 114.5) (size 0.5) (drill 0.2) (layers "F.Cu" "B.Cu") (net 15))
 (segment (start 155.5 110) (end 155.5 114.5) (width 0.2) (layer "B.Cu") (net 15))
 (segment (start 150.25 109.673) (end 150.323 109.6) (width 0.2) (layer "F.Cu") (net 16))
 (segment (start 155 109.5) (end 154.827 109.673) (width 0.2) (layer "F.Cu") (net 16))
 (segment (start 154.827 109.673) (end 150.25 109.673) (width 0.2) (layer "F.Cu") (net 16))
 (segment (start 150.323 109.6) (end 150.4625 109.6) (width 0.2) (layer "F.Cu") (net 16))
 (via (at 155 109.5) (size 0.5) (drill 0.2) (layers "F.Cu" "B.Cu") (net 16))
 (segment (start 155 109.5) (end 156 108.5) (width 0.2) (layer "B.Cu") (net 16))
 (segment (start 156 108.5) (end 158.6 108.5) (width 0.2) (layer "B.Cu") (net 16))
 (segment (start 144.75 112.25) (end 143.65 113.35) (width 0.2) (layer "F.Cu") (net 12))
 (segment (start 146.0875 112.25) (end 144.75 112.25) (width 0.2) (layer "F.Cu") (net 12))
 (segment (start 147.5375 110.8) (end 146.0875 112.25) (width 0.2) (layer "F.Cu") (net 12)))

